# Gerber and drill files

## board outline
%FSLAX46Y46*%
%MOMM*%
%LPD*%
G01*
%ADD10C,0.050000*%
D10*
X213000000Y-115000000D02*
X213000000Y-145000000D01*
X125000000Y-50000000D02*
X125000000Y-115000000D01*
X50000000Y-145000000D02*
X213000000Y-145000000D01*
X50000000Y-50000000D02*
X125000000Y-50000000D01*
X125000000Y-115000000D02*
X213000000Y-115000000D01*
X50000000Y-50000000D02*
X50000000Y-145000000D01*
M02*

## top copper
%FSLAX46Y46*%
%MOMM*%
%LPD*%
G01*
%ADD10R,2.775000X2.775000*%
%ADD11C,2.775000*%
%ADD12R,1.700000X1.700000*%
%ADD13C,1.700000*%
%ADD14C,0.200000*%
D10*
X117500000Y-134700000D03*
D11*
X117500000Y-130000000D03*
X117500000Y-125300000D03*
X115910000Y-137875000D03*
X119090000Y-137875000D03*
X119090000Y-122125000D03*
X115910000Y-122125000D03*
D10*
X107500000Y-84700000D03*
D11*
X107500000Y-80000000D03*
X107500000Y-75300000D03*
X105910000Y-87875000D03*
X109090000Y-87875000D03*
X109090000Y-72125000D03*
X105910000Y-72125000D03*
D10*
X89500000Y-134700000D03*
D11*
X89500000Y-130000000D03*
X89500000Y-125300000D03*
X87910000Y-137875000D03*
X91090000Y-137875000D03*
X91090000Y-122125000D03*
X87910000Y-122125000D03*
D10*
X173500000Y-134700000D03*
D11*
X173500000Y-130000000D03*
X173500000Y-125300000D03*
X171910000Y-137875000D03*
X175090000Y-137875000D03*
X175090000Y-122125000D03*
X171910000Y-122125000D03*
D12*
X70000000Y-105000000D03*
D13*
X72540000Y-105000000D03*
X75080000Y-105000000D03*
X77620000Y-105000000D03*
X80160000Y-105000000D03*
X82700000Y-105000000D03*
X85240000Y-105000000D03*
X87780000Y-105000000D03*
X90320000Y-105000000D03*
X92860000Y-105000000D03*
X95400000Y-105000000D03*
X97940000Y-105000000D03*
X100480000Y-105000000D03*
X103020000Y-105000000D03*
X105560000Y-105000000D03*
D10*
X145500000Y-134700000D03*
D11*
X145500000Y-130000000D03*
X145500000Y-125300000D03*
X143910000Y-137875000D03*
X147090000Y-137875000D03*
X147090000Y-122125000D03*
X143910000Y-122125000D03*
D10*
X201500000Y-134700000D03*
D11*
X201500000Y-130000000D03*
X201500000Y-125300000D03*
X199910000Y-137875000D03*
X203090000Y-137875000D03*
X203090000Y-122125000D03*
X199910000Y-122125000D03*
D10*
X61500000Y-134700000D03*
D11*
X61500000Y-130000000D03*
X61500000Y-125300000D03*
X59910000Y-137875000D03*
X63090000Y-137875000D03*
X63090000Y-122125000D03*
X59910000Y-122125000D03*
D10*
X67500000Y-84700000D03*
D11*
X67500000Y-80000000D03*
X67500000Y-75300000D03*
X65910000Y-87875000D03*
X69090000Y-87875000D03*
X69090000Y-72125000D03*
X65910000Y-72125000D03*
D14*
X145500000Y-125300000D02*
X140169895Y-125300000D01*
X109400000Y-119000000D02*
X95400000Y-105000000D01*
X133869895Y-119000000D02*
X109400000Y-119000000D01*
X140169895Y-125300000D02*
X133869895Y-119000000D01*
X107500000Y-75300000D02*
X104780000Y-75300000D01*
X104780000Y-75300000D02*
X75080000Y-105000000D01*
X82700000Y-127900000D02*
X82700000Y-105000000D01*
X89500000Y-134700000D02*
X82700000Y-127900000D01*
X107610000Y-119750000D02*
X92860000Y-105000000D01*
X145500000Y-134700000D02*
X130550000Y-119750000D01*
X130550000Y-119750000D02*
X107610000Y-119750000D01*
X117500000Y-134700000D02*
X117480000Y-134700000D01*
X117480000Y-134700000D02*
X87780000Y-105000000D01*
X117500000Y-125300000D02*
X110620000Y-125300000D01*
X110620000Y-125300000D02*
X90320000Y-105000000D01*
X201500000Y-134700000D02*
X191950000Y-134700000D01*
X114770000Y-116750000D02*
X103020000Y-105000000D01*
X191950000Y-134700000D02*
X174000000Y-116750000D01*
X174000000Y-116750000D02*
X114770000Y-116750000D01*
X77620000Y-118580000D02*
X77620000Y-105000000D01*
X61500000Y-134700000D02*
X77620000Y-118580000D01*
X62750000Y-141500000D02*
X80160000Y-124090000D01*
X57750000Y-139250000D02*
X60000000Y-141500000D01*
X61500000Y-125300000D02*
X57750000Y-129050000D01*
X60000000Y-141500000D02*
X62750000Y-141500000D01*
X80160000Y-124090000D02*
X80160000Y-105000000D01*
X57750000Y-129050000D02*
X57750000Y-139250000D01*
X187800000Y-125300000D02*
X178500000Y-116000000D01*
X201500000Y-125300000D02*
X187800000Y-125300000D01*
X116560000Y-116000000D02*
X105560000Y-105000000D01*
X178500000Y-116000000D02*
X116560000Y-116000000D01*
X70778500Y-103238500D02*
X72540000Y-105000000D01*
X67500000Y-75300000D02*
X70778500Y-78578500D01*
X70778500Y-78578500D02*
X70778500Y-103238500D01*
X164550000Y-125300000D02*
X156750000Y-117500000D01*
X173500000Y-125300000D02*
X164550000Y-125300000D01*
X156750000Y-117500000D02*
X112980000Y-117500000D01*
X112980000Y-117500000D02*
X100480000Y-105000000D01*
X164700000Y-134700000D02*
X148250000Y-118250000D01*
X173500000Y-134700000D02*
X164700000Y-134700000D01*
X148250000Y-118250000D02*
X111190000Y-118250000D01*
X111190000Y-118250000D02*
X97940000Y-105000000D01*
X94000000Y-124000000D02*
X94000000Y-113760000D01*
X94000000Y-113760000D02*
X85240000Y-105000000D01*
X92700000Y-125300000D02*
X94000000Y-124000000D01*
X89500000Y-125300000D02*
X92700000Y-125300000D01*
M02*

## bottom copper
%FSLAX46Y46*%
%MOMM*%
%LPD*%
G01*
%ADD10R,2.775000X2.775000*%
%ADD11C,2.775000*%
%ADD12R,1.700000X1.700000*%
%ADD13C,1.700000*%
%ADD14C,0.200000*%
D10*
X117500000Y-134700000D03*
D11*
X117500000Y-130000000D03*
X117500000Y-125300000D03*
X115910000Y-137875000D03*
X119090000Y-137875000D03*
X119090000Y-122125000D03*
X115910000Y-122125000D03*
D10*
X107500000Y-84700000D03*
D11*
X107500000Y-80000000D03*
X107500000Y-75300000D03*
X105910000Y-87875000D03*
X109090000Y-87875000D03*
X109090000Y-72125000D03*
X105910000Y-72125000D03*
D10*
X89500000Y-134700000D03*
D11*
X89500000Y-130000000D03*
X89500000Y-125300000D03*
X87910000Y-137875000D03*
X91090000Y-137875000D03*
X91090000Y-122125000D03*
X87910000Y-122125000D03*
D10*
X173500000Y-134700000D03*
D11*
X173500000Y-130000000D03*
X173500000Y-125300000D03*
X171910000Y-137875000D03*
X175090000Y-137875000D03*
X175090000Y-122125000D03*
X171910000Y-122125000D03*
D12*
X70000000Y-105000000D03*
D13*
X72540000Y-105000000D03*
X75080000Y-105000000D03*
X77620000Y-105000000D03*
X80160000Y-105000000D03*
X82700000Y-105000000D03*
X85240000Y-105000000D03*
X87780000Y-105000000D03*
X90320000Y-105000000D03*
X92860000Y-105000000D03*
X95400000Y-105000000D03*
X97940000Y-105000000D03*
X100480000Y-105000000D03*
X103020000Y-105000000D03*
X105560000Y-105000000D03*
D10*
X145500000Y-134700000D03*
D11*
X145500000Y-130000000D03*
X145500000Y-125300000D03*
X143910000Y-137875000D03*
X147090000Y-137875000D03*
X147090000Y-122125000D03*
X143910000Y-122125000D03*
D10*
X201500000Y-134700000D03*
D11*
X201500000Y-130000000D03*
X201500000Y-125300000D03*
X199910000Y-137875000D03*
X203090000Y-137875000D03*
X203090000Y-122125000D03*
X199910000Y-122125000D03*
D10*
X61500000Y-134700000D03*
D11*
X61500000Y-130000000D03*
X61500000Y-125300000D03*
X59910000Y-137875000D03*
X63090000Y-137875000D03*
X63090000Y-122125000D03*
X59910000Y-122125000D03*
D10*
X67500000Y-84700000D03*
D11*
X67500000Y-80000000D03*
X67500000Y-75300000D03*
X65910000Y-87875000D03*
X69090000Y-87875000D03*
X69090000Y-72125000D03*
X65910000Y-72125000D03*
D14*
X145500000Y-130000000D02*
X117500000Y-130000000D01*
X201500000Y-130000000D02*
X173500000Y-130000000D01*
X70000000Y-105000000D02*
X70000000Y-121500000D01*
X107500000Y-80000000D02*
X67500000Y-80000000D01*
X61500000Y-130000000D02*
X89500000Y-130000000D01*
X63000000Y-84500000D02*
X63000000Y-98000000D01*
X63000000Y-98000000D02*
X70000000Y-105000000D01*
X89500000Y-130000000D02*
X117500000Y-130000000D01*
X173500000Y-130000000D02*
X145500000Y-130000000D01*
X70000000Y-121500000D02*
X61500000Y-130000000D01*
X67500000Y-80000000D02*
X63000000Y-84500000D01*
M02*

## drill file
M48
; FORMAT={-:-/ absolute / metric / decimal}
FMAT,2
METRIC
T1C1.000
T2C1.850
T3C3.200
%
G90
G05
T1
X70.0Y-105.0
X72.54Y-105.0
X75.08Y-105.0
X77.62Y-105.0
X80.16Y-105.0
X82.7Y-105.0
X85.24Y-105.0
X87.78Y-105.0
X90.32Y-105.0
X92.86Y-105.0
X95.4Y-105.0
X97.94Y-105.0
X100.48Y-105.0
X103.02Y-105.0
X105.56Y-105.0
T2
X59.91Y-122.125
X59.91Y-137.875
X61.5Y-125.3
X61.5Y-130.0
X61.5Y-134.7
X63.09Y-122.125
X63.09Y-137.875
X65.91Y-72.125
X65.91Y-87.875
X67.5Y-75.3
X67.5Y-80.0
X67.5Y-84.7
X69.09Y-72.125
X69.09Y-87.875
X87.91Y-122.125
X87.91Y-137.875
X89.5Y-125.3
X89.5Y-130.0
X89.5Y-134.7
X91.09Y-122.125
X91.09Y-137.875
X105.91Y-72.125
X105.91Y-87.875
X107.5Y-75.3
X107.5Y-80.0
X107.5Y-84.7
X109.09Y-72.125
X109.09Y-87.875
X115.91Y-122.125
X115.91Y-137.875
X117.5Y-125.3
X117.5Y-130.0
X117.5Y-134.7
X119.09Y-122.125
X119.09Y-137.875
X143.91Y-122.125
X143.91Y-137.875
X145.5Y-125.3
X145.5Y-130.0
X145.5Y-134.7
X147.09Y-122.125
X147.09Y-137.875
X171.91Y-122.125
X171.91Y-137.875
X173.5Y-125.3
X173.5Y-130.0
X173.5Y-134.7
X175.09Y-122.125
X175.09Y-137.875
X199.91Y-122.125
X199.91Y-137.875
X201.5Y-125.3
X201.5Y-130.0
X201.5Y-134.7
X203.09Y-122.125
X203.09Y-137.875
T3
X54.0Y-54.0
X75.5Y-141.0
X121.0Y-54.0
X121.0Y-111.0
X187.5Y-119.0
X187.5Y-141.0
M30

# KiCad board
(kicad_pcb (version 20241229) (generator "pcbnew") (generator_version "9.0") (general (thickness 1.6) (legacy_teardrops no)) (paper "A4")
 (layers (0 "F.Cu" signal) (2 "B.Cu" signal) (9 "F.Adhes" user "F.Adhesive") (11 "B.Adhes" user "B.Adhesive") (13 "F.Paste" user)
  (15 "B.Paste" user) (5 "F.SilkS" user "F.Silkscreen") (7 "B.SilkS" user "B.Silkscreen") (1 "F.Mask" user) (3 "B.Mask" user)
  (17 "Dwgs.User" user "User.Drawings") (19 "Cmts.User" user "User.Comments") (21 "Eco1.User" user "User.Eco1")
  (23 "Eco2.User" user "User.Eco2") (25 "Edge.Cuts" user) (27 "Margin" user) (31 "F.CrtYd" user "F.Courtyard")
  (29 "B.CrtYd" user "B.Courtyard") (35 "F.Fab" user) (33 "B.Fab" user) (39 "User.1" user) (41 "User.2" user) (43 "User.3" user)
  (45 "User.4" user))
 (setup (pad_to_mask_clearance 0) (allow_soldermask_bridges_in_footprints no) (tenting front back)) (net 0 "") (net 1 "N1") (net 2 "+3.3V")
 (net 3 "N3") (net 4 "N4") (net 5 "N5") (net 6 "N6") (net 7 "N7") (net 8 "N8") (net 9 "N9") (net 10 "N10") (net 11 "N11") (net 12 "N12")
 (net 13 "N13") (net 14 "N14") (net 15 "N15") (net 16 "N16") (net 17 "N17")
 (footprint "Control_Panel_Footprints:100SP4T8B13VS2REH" (layer "F.Cu") (at 117.5 134.7 90)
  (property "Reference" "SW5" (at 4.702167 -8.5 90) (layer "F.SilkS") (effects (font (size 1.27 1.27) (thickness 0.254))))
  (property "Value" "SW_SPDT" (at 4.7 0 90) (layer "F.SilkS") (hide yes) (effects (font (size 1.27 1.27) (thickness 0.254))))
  (pad "1" thru_hole rect (at 0 0 90) (size 2.775 2.775) (drill 1.85) (layers "*.Cu" "*.Mask") (remove_unused_layers no) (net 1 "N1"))
  (pad "2" thru_hole circle (at 4.7 0 90) (size 2.775 2.775) (drill 1.85) (layers "*.Cu" "*.Mask") (remove_unused_layers no) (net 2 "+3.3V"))
  (pad "3" thru_hole circle (at 9.4 0 90) (size 2.775 2.775) (drill 1.85) (layers "*.Cu" "*.Mask") (remove_unused_layers no) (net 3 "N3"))
  (pad "4" thru_hole circle (at -3.175 -1.59 90) (size 2.775 2.775) (drill 1.85) (layers "*.Cu" "*.Mask") (remove_unused_layers no))
  (pad "5" thru_hole circle (at -3.175 1.59 90) (size 2.775 2.775) (drill 1.85) (layers "*.Cu" "*.Mask") (remove_unused_layers no))
  (pad "6" thru_hole circle (at 12.575 1.59 90) (size 2.775 2.775) (drill 1.85) (layers "*.Cu" "*.Mask") (remove_unused_layers no))
  (pad "7" thru_hole circle (at 12.575 -1.59 90) (size 2.775 2.775) (drill 1.85) (layers "*.Cu" "*.Mask") (remove_unused_layers no)))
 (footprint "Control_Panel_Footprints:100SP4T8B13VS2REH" (layer "F.Cu") (at 107.5 84.7 90)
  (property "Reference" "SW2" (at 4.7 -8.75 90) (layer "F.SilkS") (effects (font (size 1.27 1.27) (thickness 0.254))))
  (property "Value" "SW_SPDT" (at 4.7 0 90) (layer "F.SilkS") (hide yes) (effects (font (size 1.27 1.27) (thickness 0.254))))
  (pad "1" thru_hole rect (at 0 0 90) (size 2.775 2.775) (drill 1.85) (layers "*.Cu" "*.Mask") (remove_unused_layers no) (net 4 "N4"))
  (pad "2" thru_hole circle (at 4.7 0 90) (size 2.775 2.775) (drill 1.85) (layers "*.Cu" "*.Mask") (remove_unused_layers no) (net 2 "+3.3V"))
  (pad "3" thru_hole circle (at 9.4 0 90) (size 2.775 2.775) (drill 1.85) (layers "*.Cu" "*.Mask") (remove_unused_layers no) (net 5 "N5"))
  (pad "4" thru_hole circle (at -3.175 -1.59 90) (size 2.775 2.775) (drill 1.85) (layers "*.Cu" "*.Mask") (remove_unused_layers no))
  (pad "5" thru_hole circle (at -3.175 1.59 90) (size 2.775 2.775) (drill 1.85) (layers "*.Cu" "*.Mask") (remove_unused_layers no))
  (pad "6" thru_hole circle (at 12.575 1.59 90) (size 2.775 2.775) (drill 1.85) (layers "*.Cu" "*.Mask") (remove_unused_layers no))
  (pad "7" thru_hole circle (at 12.575 -1.59 90) (size 2.775 2.775) (drill 1.85) (layers "*.Cu" "*.Mask") (remove_unused_layers no)))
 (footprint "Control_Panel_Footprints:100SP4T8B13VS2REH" (layer "F.Cu") (at 89.5 134.7 90)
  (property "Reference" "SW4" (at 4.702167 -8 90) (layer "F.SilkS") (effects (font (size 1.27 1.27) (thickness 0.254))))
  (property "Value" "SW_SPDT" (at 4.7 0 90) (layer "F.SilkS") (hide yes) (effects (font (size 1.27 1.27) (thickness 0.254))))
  (pad "1" thru_hole rect (at 0 0 90) (size 2.775 2.775) (drill 1.85) (layers "*.Cu" "*.Mask") (remove_unused_layers no) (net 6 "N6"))
  (pad "2" thru_hole circle (at 4.7 0 90) (size 2.775 2.775) (drill 1.85) (layers "*.Cu" "*.Mask") (remove_unused_layers no) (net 2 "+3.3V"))
  (pad "3" thru_hole circle (at 9.4 0 90) (size 2.775 2.775) (drill 1.85) (layers "*.Cu" "*.Mask") (remove_unused_layers no) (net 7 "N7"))
  (pad "4" thru_hole circle (at -3.175 -1.59 90) (size 2.775 2.775) (drill 1.85) (layers "*.Cu" "*.Mask") (remove_unused_layers no))
  (pad "5" thru_hole circle (at -3.175 1.59 90) (size 2.775 2.775) (drill 1.85) (layers "*.Cu" "*.Mask") (remove_unused_layers no))
  (pad "6" thru_hole circle (at 12.575 1.59 90) (size 2.775 2.775) (drill 1.85) (layers "*.Cu" "*.Mask") (remove_unused_layers no))
  (pad "7" thru_hole circle (at 12.575 -1.59 90) (size 2.775 2.775) (drill 1.85) (layers "*.Cu" "*.Mask") (remove_unused_layers no)))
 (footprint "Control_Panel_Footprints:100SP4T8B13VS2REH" (layer "F.Cu") (at 173.5 134.7 90)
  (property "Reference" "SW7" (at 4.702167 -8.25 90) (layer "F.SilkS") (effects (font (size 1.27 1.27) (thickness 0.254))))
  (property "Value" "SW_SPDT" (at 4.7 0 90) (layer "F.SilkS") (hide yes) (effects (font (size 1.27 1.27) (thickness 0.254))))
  (pad "1" thru_hole rect (at 0 0 90) (size 2.775 2.775) (drill 1.85) (layers "*.Cu" "*.Mask") (remove_unused_layers no) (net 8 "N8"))
  (pad "2" thru_hole circle (at 4.7 0 90) (size 2.775 2.775) (drill 1.85) (layers "*.Cu" "*.Mask") (remove_unused_layers no) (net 2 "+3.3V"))
  (pad "3" thru_hole circle (at 9.4 0 90) (size 2.775 2.775) (drill 1.85) (layers "*.Cu" "*.Mask") (remove_unused_layers no) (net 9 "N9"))
  (pad "4" thru_hole circle (at -3.175 -1.59 90) (size 2.775 2.775) (drill 1.85) (layers "*.Cu" "*.Mask") (remove_unused_layers no))
  (pad "5" thru_hole circle (at -3.175 1.59 90) (size 2.775 2.775) (drill 1.85) (layers "*.Cu" "*.Mask") (remove_unused_layers no))
  (pad "6" thru_hole circle (at 12.575 1.59 90) (size 2.775 2.775) (drill 1.85) (layers "*.Cu" "*.Mask") (remove_unused_layers no))
  (pad "7" thru_hole circle (at 12.575 -1.59 90) (size 2.775 2.775) (drill 1.85) (layers "*.Cu" "*.Mask") (remove_unused_layers no)))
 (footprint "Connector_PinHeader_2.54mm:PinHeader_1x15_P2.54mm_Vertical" (layer "F.Cu") (at 70 105 90)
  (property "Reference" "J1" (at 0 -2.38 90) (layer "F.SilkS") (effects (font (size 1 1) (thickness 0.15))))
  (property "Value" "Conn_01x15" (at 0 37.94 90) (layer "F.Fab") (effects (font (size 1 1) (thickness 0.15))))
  (pad "1" thru_hole rect (at 0 0 90) (size 1.7 1.7) (drill 1) (layers "*.Cu" "*.Mask") (remove_unused_layers no) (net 2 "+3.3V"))
  (pad "2" thru_hole circle (at 0 2.54 90) (size 1.7 1.7) (drill 1) (layers "*.Cu" "*.Mask") (remove_unused_layers no) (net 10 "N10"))
  (pad "3" thru_hole circle (at 0 5.08 90) (size 1.7 1.7) (drill 1) (layers "*.Cu" "*.Mask") (remove_unused_layers no) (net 5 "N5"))
  (pad "4" thru_hole circle (at 0 7.62 90) (size 1.7 1.7) (drill 1) (layers "*.Cu" "*.Mask") (remove_unused_layers no) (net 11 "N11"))
  (pad "5" thru_hole circle (at 0 10.16 90) (size 1.7 1.7) (drill 1) (layers "*.Cu" "*.Mask") (remove_unused_layers no) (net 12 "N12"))
  (pad "6" thru_hole circle (at 0 12.7 90) (size 1.7 1.7) (drill 1) (layers "*.Cu" "*.Mask") (remove_unused_layers no) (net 6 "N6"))
  (pad "7" thru_hole circle (at 0 15.24 90) (size 1.7 1.7) (drill 1) (layers "*.Cu" "*.Mask") (remove_unused_layers no) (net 7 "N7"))
  (pad "8" thru_hole circle (at 0 17.78 90) (size 1.7 1.7) (drill 1) (layers "*.Cu" "*.Mask") (remove_unused_layers no) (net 1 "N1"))
  (pad "9" thru_hole circle (at 0 20.32 90) (size 1.7 1.7) (drill 1) (layers "*.Cu" "*.Mask") (remove_unused_layers no) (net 3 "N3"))
  (pad "10" thru_hole circle (at 0 22.86 90) (size 1.7 1.7) (drill 1) (layers "*.Cu" "*.Mask") (remove_unused_layers no) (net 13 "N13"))
  (pad "11" thru_hole circle (at 0 25.4 90) (size 1.7 1.7) (drill 1) (layers "*.Cu" "*.Mask") (remove_unused_layers no) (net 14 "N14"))
  (pad "12" thru_hole circle (at 0 27.94 90) (size 1.7 1.7) (drill 1) (layers "*.Cu" "*.Mask") (remove_unused_layers no) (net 8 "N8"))
  (pad "13" thru_hole circle (at 0 30.48 90) (size 1.7 1.7) (drill 1) (layers "*.Cu" "*.Mask") (remove_unused_layers no) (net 9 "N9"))
  (pad "14" thru_hole circle (at 0 33.02 90) (size 1.7 1.7) (drill 1) (layers "*.Cu" "*.Mask") (remove_unused_layers no) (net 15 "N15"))
  (pad "15" thru_hole circle (at 0 35.56 90) (size 1.7 1.7) (drill 1) (layers "*.Cu" "*.Mask") (remove_unused_layers no) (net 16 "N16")))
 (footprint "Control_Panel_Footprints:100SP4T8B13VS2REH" (layer "F.Cu") (at 145.5 134.7 90)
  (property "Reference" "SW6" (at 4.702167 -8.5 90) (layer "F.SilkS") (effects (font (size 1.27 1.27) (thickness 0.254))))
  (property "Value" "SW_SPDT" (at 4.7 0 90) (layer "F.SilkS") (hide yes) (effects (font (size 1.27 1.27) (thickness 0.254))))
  (pad "1" thru_hole rect (at 0 0 90) (size 2.775 2.775) (drill 1.85) (layers "*.Cu" "*.Mask") (remove_unused_layers no) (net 13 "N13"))
  (pad "2" thru_hole circle (at 4.7 0 90) (size 2.775 2.775) (drill 1.85) (layers "*.Cu" "*.Mask") (remove_unused_layers no) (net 2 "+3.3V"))
  (pad "3" thru_hole circle (at 9.4 0 90) (size 2.775 2.775) (drill 1.85) (layers "*.Cu" "*.Mask") (remove_unused_layers no) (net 14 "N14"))
  (pad "4" thru_hole circle (at -3.175 -1.59 90) (size 2.775 2.775) (drill 1.85) (layers "*.Cu" "*.Mask") (remove_unused_layers no))
  (pad "5" thru_hole circle (at -3.175 1.59 90) (size 2.775 2.775) (drill 1.85) (layers "*.Cu" "*.Mask") (remove_unused_layers no))
  (pad "6" thru_hole circle (at 12.575 1.59 90) (size 2.775 2.775) (drill 1.85) (layers "*.Cu" "*.Mask") (remove_unused_layers no))
  (pad "7" thru_hole circle (at 12.575 -1.59 90) (size 2.775 2.775) (drill 1.85) (layers "*.Cu" "*.Mask") (remove_unused_layers no)))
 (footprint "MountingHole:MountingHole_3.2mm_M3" (layer "F.Cu") (at 187.5 141)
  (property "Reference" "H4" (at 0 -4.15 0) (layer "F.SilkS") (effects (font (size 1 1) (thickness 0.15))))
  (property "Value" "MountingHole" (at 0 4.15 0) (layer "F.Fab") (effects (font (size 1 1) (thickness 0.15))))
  (pad "" np_thru_hole circle (at 0 0) (size 3.2 3.2) (drill 3.2) (layers "*.Cu" "*.Mask")))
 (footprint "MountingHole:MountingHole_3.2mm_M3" (layer "F.Cu") (at 75.5 141)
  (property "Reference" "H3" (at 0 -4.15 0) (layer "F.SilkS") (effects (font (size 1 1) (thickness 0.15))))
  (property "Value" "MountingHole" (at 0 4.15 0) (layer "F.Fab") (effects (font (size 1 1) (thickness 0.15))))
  (pad "" np_thru_hole circle (at 0 0) (size 3.2 3.2) (drill 3.2) (layers "*.Cu" "*.Mask")))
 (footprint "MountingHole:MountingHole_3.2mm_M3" (layer "F.Cu") (at 121 111)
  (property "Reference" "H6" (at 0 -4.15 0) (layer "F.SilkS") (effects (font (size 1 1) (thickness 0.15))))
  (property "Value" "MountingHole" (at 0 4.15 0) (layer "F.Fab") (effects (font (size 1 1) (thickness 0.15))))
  (pad "" np_thru_hole circle (at 0 0) (size 3.2 3.2) (drill 3.2) (layers "*.Cu" "*.Mask")))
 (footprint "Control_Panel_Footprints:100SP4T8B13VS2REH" (layer "F.Cu") (at 201.5 134.7 90)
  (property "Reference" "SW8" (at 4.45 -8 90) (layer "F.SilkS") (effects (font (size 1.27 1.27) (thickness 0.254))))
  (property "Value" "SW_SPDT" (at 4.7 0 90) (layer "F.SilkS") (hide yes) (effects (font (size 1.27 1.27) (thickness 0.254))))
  (pad "1" thru_hole rect (at 0 0 90) (size 2.775 2.775) (drill 1.85) (layers "*.Cu" "*.Mask") (remove_unused_layers no) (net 15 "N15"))
  (pad "2" thru_hole circle (at 4.7 0 90) (size 2.775 2.775) (drill 1.85) (layers "*.Cu" "*.Mask") (remove_unused_layers no) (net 2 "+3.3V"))
  (pad "3" thru_hole circle (at 9.4 0 90) (size 2.775 2.775) (drill 1.85) (layers "*.Cu" "*.Mask") (remove_unused_layers no) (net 16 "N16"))
  (pad "4" thru_hole circle (at -3.175 -1.59 90) (size 2.775 2.775) (drill 1.85) (layers "*.Cu" "*.Mask") (remove_unused_layers no))
  (pad "5" thru_hole circle (at -3.175 1.59 90) (size 2.775 2.775) (drill 1.85) (layers "*.Cu" "*.Mask") (remove_unused_layers no))
  (pad "6" thru_hole circle (at 12.575 1.59 90) (size 2.775 2.775) (drill 1.85) (layers "*.Cu" "*.Mask") (remove_unused_layers no))
  (pad "7" thru_hole circle (at 12.575 -1.59 90) (size 2.775 2.775) (drill 1.85) (layers "*.Cu" "*.Mask") (remove_unused_layers no)))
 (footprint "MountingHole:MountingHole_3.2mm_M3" (layer "F.Cu") (at 54 54)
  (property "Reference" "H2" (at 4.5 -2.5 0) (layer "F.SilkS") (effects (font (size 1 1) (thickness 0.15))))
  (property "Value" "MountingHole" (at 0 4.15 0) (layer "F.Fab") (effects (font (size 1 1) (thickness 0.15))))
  (pad "" np_thru_hole circle (at 0 0) (size 3.2 3.2) (drill 3.2) (layers "*.Cu" "*.Mask")))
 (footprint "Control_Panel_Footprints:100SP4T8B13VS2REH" (layer "F.Cu") (at 61.5 134.7 90)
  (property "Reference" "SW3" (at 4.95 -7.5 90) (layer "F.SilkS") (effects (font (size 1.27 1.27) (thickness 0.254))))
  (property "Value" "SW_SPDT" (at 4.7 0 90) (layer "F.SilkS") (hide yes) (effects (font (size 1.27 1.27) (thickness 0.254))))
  (pad "1" thru_hole rect (at 0 0 90) (size 2.775 2.775) (drill 1.85) (layers "*.Cu" "*.Mask") (remove_unused_layers no) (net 11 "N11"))
  (pad "2" thru_hole circle (at 4.7 0 90) (size 2.775 2.775) (drill 1.85) (layers "*.Cu" "*.Mask") (remove_unused_layers no) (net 2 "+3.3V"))
  (pad "3" thru_hole circle (at 9.4 0 90) (size 2.775 2.775) (drill 1.85) (layers "*.Cu" "*.Mask") (remove_unused_layers no) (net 12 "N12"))
  (pad "4" thru_hole circle (at -3.175 -1.59 90) (size 2.775 2.775) (drill 1.85) (layers "*.Cu" "*.Mask") (remove_unused_layers no))
  (pad "5" thru_hole circle (at -3.175 1.59 90) (size 2.775 2.775) (drill 1.85) (layers "*.Cu" "*.Mask") (remove_unused_layers no))
  (pad "6" thru_hole circle (at 12.575 1.59 90) (size 2.775 2.775) (drill 1.85) (layers "*.Cu" "*.Mask") (remove_unused_layers no))
  (pad "7" thru_hole circle (at 12.575 -1.59 90) (size 2.775 2.775) (drill 1.85) (layers "*.Cu" "*.Mask") (remove_unused_layers no)))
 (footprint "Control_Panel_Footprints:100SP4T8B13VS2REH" (layer "F.Cu") (at 67.5 84.7 90)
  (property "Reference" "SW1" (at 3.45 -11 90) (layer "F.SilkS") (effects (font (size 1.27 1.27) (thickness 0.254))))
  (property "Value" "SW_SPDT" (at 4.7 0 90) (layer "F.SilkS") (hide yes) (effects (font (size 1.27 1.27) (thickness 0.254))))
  (pad "1" thru_hole rect (at 0 0 90) (size 2.775 2.775) (drill 1.85) (layers "*.Cu" "*.Mask") (remove_unused_layers no) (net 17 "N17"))
  (pad "2" thru_hole circle (at 4.7 0 90) (size 2.775 2.775) (drill 1.85) (layers "*.Cu" "*.Mask") (remove_unused_layers no) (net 2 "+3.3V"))
  (pad "3" thru_hole circle (at 9.4 0 90) (size 2.775 2.775) (drill 1.85) (layers "*.Cu" "*.Mask") (remove_unused_layers no) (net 10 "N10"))
  (pad "4" thru_hole circle (at -3.175 -1.59 90) (size 2.775 2.775) (drill 1.85) (layers "*.Cu" "*.Mask") (remove_unused_layers no))
  (pad "5" thru_hole circle (at -3.175 1.59 90) (size 2.775 2.775) (drill 1.85) (layers "*.Cu" "*.Mask") (remove_unused_layers no))
  (pad "6" thru_hole circle (at 12.575 1.59 90) (size 2.775 2.775) (drill 1.85) (layers "*.Cu" "*.Mask") (remove_unused_layers no))
  (pad "7" thru_hole circle (at 12.575 -1.59 90) (size 2.775 2.775) (drill 1.85) (layers "*.Cu" "*.Mask") (remove_unused_layers no)))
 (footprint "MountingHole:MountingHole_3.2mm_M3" (layer "F.Cu") (at 187.5 119)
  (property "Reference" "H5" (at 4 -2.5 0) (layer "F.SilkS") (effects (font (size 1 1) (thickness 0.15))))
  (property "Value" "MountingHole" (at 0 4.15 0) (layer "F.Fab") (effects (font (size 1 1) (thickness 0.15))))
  (pad "" np_thru_hole circle (at 0 0) (size 3.2 3.2) (drill 3.2) (layers "*.Cu" "*.Mask")))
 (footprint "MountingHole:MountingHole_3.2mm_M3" (layer "F.Cu") (at 121 54)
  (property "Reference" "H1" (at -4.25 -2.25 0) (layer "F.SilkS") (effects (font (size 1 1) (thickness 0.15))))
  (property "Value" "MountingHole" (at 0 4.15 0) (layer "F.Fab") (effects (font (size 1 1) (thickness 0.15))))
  (pad "" np_thru_hole circle (at 0 0) (size 3.2 3.2) (drill 3.2) (layers "*.Cu" "*.Mask")))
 (gr_line (start 213 115) (end 213 145) (stroke (width 0.05) (type default)) (layer "Edge.Cuts"))
 (gr_line (start 125 50) (end 125 115) (stroke (width 0.05) (type solid)) (layer "Edge.Cuts"))
 (gr_line (start 50 145) (end 213 145) (stroke (width 0.05) (type solid)) (layer "Edge.Cuts"))
 (gr_line (start 50 50) (end 125 50) (stroke (width 0.05) (type solid)) (layer "Edge.Cuts"))
 (gr_line (start 125 115) (end 213 115) (stroke (width 0.05) (type solid)) (layer "Edge.Cuts"))
 (gr_line (start 50 50) (end 50 145) (stroke (width 0.05) (type solid)) (layer "Edge.Cuts"))
 (segment (start 145.5 125.3) (end 140.169895 125.3) (width 0.2) (layer "F.Cu") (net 14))
 (segment (start 109.4 119) (end 95.4 105) (width 0.2) (layer "F.Cu") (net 14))
 (segment (start 133.869895 119) (end 109.4 119) (width 0.2) (layer "F.Cu") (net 14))
 (segment (start 140.169895 125.3) (end 133.869895 119) (width 0.2) (layer "F.Cu") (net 14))
 (segment (start 107.5 75.3) (end 104.78 75.3) (width 0.2) (layer "F.Cu") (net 5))
 (segment (start 104.78 75.3) (end 75.08 105) (width 0.2) (layer "F.Cu") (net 5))
 (segment (start 82.7 127.9) (end 82.7 105) (width 0.2) (layer "F.Cu") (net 6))
 (segment (start 89.5 134.7) (end 82.7 127.9) (width 0.2) (layer "F.Cu") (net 6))
 (segment (start 145.5 130) (end 117.5 130) (width 0.2) (layer "B.Cu") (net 2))
 (segment (start 201.5 130) (end 173.5 130) (width 0.2) (layer "B.Cu") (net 2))
 (segment (start 70 105) (end 70 121.5) (width 0.2) (layer "B.Cu") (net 2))
 (segment (start 107.5 80) (end 67.5 80) (width 0.2) (layer "B.Cu") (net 2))
 (segment (start 61.5 130) (end 89.5 130) (width 0.2) (layer "B.Cu") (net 2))
 (segment (start 63 84.5) (end 63 98) (width 0.2) (layer "B.Cu") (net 2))
 (segment (start 63 98) (end 70 105) (width 0.2) (layer "B.Cu") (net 2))
 (segment (start 89.5 130) (end 117.5 130) (width 0.2) (layer "B.Cu") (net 2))
 (segment (start 173.5 130) (end 145.5 130) (width 0.2) (layer "B.Cu") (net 2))
 (segment (start 70 121.5) (end 61.5 130) (width 0.2) (layer "B.Cu") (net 2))
 (segment (start 67.5 80) (end 63 84.5) (width 0.2) (layer "B.Cu") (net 2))
 (segment (start 107.61 119.75) (end 92.86 105) (width 0.2) (layer "F.Cu") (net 13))
 (segment (start 145.5 134.7) (end 130.55 119.75) (width 0.2) (layer "F.Cu") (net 13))
 (segment (start 130.55 119.75) (end 107.61 119.75) (width 0.2) (layer "F.Cu") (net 13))
 (segment (start 117.5 134.7) (end 117.48 134.7) (width 0.2) (layer "F.Cu") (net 1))
 (segment (start 117.48 134.7) (end 87.78 105) (width 0.2) (layer "F.Cu") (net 1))
 (segment (start 117.5 125.3) (end 110.62 125.3) (width 0.2) (layer "F.Cu") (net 3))
 (segment (start 110.62 125.3) (end 90.32 105) (width 0.2) (layer "F.Cu") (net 3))
 (segment (start 201.5 134.7) (end 191.95 134.7) (width 0.2) (layer "F.Cu") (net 15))
 (segment (start 114.77 116.75) (end 103.02 105) (width 0.2) (layer "F.Cu") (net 15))
 (segment (start 191.95 134.7) (end 174 116.75) (width 0.2) (layer "F.Cu") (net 15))
 (segment (start 174 116.75) (end 114.77 116.75) (width 0.2) (layer "F.Cu") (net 15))
 (segment (start 77.62 118.58) (end 77.62 105) (width 0.2) (layer "F.Cu") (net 11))
 (segment (start 61.5 134.7) (end 77.62 118.58) (width 0.2) (layer "F.Cu") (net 11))
 (segment (start 62.75 141.5) (end 80.16 124.09) (width 0.2) (layer "F.Cu") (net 12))
 (segment (start 57.75 139.25) (end 60 141.5) (width 0.2) (layer "F.Cu") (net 12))
 (segment (start 61.5 125.3) (end 57.75 129.05) (width 0.2) (layer "F.Cu") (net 12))
 (segment (start 60 141.5) (end 62.75 141.5) (width 0.2) (layer "F.Cu") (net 12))
 (segment (start 80.16 124.09) (end 80.16 105) (width 0.2) (layer "F.Cu") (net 12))
 (segment (start 57.75 129.05) (end 57.75 139.25) (width 0.2) (layer "F.Cu") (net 12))
 (segment (start 187.8 125.3) (end 178.5 116) (width 0.2) (layer "F.Cu") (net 16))
 (segment (start 201.5 125.3) (end 187.8 125.3) (width 0.2) (layer "F.Cu") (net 16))
 (segment (start 116.56 116) (end 105.56 105) (width 0.2) (layer "F.Cu") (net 16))
 (segment (start 178.5 116) (end 116.56 116) (width 0.2) (layer "F.Cu") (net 16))
 (segment (start 70.7785 103.2385) (end 72.54 105) (width 0.2) (layer "F.Cu") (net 10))
 (segment (start 67.5 75.3) (end 70.7785 78.5785) (width 0.2) (layer "F.Cu") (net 10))
 (segment (start 70.7785 78.5785) (end 70.7785 103.2385) (width 0.2) (layer "F.Cu") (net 10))
 (segment (start 164.55 125.3) (end 156.75 117.5) (width 0.2) (layer "F.Cu") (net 9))
 (segment (start 173.5 125.3) (end 164.55 125.3) (width 0.2) (layer "F.Cu") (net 9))
 (segment (start 156.75 117.5) (end 112.98 117.5) (width 0.2) (layer "F.Cu") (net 9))
 (segment (start 112.98 117.5) (end 100.48 105) (width 0.2) (layer "F.Cu") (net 9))
 (segment (start 164.7 134.7) (end 148.25 118.25) (width 0.2) (layer "F.Cu") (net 8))
 (segment (start 173.5 134.7) (end 164.7 134.7) (width 0.2) (layer "F.Cu") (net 8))
 (segment (start 148.25 118.25) (end 111.19 118.25) (width 0.2) (layer "F.Cu") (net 8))
 (segment (start 111.19 118.25) (end 97.94 105) (width 0.2) (layer "F.Cu") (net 8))
 (segment (start 94 124) (end 94 113.76) (width 0.2) (layer "F.Cu") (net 7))
 (segment (start 94 113.76) (end 85.24 105) (width 0.2) (layer "F.Cu") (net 7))
 (segment (start 92.7 125.3) (end 94 124) (width 0.2) (layer "F.Cu") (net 7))
 (segment (start 89.5 125.3) (end 92.7 125.3) (width 0.2) (layer "F.Cu") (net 7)))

